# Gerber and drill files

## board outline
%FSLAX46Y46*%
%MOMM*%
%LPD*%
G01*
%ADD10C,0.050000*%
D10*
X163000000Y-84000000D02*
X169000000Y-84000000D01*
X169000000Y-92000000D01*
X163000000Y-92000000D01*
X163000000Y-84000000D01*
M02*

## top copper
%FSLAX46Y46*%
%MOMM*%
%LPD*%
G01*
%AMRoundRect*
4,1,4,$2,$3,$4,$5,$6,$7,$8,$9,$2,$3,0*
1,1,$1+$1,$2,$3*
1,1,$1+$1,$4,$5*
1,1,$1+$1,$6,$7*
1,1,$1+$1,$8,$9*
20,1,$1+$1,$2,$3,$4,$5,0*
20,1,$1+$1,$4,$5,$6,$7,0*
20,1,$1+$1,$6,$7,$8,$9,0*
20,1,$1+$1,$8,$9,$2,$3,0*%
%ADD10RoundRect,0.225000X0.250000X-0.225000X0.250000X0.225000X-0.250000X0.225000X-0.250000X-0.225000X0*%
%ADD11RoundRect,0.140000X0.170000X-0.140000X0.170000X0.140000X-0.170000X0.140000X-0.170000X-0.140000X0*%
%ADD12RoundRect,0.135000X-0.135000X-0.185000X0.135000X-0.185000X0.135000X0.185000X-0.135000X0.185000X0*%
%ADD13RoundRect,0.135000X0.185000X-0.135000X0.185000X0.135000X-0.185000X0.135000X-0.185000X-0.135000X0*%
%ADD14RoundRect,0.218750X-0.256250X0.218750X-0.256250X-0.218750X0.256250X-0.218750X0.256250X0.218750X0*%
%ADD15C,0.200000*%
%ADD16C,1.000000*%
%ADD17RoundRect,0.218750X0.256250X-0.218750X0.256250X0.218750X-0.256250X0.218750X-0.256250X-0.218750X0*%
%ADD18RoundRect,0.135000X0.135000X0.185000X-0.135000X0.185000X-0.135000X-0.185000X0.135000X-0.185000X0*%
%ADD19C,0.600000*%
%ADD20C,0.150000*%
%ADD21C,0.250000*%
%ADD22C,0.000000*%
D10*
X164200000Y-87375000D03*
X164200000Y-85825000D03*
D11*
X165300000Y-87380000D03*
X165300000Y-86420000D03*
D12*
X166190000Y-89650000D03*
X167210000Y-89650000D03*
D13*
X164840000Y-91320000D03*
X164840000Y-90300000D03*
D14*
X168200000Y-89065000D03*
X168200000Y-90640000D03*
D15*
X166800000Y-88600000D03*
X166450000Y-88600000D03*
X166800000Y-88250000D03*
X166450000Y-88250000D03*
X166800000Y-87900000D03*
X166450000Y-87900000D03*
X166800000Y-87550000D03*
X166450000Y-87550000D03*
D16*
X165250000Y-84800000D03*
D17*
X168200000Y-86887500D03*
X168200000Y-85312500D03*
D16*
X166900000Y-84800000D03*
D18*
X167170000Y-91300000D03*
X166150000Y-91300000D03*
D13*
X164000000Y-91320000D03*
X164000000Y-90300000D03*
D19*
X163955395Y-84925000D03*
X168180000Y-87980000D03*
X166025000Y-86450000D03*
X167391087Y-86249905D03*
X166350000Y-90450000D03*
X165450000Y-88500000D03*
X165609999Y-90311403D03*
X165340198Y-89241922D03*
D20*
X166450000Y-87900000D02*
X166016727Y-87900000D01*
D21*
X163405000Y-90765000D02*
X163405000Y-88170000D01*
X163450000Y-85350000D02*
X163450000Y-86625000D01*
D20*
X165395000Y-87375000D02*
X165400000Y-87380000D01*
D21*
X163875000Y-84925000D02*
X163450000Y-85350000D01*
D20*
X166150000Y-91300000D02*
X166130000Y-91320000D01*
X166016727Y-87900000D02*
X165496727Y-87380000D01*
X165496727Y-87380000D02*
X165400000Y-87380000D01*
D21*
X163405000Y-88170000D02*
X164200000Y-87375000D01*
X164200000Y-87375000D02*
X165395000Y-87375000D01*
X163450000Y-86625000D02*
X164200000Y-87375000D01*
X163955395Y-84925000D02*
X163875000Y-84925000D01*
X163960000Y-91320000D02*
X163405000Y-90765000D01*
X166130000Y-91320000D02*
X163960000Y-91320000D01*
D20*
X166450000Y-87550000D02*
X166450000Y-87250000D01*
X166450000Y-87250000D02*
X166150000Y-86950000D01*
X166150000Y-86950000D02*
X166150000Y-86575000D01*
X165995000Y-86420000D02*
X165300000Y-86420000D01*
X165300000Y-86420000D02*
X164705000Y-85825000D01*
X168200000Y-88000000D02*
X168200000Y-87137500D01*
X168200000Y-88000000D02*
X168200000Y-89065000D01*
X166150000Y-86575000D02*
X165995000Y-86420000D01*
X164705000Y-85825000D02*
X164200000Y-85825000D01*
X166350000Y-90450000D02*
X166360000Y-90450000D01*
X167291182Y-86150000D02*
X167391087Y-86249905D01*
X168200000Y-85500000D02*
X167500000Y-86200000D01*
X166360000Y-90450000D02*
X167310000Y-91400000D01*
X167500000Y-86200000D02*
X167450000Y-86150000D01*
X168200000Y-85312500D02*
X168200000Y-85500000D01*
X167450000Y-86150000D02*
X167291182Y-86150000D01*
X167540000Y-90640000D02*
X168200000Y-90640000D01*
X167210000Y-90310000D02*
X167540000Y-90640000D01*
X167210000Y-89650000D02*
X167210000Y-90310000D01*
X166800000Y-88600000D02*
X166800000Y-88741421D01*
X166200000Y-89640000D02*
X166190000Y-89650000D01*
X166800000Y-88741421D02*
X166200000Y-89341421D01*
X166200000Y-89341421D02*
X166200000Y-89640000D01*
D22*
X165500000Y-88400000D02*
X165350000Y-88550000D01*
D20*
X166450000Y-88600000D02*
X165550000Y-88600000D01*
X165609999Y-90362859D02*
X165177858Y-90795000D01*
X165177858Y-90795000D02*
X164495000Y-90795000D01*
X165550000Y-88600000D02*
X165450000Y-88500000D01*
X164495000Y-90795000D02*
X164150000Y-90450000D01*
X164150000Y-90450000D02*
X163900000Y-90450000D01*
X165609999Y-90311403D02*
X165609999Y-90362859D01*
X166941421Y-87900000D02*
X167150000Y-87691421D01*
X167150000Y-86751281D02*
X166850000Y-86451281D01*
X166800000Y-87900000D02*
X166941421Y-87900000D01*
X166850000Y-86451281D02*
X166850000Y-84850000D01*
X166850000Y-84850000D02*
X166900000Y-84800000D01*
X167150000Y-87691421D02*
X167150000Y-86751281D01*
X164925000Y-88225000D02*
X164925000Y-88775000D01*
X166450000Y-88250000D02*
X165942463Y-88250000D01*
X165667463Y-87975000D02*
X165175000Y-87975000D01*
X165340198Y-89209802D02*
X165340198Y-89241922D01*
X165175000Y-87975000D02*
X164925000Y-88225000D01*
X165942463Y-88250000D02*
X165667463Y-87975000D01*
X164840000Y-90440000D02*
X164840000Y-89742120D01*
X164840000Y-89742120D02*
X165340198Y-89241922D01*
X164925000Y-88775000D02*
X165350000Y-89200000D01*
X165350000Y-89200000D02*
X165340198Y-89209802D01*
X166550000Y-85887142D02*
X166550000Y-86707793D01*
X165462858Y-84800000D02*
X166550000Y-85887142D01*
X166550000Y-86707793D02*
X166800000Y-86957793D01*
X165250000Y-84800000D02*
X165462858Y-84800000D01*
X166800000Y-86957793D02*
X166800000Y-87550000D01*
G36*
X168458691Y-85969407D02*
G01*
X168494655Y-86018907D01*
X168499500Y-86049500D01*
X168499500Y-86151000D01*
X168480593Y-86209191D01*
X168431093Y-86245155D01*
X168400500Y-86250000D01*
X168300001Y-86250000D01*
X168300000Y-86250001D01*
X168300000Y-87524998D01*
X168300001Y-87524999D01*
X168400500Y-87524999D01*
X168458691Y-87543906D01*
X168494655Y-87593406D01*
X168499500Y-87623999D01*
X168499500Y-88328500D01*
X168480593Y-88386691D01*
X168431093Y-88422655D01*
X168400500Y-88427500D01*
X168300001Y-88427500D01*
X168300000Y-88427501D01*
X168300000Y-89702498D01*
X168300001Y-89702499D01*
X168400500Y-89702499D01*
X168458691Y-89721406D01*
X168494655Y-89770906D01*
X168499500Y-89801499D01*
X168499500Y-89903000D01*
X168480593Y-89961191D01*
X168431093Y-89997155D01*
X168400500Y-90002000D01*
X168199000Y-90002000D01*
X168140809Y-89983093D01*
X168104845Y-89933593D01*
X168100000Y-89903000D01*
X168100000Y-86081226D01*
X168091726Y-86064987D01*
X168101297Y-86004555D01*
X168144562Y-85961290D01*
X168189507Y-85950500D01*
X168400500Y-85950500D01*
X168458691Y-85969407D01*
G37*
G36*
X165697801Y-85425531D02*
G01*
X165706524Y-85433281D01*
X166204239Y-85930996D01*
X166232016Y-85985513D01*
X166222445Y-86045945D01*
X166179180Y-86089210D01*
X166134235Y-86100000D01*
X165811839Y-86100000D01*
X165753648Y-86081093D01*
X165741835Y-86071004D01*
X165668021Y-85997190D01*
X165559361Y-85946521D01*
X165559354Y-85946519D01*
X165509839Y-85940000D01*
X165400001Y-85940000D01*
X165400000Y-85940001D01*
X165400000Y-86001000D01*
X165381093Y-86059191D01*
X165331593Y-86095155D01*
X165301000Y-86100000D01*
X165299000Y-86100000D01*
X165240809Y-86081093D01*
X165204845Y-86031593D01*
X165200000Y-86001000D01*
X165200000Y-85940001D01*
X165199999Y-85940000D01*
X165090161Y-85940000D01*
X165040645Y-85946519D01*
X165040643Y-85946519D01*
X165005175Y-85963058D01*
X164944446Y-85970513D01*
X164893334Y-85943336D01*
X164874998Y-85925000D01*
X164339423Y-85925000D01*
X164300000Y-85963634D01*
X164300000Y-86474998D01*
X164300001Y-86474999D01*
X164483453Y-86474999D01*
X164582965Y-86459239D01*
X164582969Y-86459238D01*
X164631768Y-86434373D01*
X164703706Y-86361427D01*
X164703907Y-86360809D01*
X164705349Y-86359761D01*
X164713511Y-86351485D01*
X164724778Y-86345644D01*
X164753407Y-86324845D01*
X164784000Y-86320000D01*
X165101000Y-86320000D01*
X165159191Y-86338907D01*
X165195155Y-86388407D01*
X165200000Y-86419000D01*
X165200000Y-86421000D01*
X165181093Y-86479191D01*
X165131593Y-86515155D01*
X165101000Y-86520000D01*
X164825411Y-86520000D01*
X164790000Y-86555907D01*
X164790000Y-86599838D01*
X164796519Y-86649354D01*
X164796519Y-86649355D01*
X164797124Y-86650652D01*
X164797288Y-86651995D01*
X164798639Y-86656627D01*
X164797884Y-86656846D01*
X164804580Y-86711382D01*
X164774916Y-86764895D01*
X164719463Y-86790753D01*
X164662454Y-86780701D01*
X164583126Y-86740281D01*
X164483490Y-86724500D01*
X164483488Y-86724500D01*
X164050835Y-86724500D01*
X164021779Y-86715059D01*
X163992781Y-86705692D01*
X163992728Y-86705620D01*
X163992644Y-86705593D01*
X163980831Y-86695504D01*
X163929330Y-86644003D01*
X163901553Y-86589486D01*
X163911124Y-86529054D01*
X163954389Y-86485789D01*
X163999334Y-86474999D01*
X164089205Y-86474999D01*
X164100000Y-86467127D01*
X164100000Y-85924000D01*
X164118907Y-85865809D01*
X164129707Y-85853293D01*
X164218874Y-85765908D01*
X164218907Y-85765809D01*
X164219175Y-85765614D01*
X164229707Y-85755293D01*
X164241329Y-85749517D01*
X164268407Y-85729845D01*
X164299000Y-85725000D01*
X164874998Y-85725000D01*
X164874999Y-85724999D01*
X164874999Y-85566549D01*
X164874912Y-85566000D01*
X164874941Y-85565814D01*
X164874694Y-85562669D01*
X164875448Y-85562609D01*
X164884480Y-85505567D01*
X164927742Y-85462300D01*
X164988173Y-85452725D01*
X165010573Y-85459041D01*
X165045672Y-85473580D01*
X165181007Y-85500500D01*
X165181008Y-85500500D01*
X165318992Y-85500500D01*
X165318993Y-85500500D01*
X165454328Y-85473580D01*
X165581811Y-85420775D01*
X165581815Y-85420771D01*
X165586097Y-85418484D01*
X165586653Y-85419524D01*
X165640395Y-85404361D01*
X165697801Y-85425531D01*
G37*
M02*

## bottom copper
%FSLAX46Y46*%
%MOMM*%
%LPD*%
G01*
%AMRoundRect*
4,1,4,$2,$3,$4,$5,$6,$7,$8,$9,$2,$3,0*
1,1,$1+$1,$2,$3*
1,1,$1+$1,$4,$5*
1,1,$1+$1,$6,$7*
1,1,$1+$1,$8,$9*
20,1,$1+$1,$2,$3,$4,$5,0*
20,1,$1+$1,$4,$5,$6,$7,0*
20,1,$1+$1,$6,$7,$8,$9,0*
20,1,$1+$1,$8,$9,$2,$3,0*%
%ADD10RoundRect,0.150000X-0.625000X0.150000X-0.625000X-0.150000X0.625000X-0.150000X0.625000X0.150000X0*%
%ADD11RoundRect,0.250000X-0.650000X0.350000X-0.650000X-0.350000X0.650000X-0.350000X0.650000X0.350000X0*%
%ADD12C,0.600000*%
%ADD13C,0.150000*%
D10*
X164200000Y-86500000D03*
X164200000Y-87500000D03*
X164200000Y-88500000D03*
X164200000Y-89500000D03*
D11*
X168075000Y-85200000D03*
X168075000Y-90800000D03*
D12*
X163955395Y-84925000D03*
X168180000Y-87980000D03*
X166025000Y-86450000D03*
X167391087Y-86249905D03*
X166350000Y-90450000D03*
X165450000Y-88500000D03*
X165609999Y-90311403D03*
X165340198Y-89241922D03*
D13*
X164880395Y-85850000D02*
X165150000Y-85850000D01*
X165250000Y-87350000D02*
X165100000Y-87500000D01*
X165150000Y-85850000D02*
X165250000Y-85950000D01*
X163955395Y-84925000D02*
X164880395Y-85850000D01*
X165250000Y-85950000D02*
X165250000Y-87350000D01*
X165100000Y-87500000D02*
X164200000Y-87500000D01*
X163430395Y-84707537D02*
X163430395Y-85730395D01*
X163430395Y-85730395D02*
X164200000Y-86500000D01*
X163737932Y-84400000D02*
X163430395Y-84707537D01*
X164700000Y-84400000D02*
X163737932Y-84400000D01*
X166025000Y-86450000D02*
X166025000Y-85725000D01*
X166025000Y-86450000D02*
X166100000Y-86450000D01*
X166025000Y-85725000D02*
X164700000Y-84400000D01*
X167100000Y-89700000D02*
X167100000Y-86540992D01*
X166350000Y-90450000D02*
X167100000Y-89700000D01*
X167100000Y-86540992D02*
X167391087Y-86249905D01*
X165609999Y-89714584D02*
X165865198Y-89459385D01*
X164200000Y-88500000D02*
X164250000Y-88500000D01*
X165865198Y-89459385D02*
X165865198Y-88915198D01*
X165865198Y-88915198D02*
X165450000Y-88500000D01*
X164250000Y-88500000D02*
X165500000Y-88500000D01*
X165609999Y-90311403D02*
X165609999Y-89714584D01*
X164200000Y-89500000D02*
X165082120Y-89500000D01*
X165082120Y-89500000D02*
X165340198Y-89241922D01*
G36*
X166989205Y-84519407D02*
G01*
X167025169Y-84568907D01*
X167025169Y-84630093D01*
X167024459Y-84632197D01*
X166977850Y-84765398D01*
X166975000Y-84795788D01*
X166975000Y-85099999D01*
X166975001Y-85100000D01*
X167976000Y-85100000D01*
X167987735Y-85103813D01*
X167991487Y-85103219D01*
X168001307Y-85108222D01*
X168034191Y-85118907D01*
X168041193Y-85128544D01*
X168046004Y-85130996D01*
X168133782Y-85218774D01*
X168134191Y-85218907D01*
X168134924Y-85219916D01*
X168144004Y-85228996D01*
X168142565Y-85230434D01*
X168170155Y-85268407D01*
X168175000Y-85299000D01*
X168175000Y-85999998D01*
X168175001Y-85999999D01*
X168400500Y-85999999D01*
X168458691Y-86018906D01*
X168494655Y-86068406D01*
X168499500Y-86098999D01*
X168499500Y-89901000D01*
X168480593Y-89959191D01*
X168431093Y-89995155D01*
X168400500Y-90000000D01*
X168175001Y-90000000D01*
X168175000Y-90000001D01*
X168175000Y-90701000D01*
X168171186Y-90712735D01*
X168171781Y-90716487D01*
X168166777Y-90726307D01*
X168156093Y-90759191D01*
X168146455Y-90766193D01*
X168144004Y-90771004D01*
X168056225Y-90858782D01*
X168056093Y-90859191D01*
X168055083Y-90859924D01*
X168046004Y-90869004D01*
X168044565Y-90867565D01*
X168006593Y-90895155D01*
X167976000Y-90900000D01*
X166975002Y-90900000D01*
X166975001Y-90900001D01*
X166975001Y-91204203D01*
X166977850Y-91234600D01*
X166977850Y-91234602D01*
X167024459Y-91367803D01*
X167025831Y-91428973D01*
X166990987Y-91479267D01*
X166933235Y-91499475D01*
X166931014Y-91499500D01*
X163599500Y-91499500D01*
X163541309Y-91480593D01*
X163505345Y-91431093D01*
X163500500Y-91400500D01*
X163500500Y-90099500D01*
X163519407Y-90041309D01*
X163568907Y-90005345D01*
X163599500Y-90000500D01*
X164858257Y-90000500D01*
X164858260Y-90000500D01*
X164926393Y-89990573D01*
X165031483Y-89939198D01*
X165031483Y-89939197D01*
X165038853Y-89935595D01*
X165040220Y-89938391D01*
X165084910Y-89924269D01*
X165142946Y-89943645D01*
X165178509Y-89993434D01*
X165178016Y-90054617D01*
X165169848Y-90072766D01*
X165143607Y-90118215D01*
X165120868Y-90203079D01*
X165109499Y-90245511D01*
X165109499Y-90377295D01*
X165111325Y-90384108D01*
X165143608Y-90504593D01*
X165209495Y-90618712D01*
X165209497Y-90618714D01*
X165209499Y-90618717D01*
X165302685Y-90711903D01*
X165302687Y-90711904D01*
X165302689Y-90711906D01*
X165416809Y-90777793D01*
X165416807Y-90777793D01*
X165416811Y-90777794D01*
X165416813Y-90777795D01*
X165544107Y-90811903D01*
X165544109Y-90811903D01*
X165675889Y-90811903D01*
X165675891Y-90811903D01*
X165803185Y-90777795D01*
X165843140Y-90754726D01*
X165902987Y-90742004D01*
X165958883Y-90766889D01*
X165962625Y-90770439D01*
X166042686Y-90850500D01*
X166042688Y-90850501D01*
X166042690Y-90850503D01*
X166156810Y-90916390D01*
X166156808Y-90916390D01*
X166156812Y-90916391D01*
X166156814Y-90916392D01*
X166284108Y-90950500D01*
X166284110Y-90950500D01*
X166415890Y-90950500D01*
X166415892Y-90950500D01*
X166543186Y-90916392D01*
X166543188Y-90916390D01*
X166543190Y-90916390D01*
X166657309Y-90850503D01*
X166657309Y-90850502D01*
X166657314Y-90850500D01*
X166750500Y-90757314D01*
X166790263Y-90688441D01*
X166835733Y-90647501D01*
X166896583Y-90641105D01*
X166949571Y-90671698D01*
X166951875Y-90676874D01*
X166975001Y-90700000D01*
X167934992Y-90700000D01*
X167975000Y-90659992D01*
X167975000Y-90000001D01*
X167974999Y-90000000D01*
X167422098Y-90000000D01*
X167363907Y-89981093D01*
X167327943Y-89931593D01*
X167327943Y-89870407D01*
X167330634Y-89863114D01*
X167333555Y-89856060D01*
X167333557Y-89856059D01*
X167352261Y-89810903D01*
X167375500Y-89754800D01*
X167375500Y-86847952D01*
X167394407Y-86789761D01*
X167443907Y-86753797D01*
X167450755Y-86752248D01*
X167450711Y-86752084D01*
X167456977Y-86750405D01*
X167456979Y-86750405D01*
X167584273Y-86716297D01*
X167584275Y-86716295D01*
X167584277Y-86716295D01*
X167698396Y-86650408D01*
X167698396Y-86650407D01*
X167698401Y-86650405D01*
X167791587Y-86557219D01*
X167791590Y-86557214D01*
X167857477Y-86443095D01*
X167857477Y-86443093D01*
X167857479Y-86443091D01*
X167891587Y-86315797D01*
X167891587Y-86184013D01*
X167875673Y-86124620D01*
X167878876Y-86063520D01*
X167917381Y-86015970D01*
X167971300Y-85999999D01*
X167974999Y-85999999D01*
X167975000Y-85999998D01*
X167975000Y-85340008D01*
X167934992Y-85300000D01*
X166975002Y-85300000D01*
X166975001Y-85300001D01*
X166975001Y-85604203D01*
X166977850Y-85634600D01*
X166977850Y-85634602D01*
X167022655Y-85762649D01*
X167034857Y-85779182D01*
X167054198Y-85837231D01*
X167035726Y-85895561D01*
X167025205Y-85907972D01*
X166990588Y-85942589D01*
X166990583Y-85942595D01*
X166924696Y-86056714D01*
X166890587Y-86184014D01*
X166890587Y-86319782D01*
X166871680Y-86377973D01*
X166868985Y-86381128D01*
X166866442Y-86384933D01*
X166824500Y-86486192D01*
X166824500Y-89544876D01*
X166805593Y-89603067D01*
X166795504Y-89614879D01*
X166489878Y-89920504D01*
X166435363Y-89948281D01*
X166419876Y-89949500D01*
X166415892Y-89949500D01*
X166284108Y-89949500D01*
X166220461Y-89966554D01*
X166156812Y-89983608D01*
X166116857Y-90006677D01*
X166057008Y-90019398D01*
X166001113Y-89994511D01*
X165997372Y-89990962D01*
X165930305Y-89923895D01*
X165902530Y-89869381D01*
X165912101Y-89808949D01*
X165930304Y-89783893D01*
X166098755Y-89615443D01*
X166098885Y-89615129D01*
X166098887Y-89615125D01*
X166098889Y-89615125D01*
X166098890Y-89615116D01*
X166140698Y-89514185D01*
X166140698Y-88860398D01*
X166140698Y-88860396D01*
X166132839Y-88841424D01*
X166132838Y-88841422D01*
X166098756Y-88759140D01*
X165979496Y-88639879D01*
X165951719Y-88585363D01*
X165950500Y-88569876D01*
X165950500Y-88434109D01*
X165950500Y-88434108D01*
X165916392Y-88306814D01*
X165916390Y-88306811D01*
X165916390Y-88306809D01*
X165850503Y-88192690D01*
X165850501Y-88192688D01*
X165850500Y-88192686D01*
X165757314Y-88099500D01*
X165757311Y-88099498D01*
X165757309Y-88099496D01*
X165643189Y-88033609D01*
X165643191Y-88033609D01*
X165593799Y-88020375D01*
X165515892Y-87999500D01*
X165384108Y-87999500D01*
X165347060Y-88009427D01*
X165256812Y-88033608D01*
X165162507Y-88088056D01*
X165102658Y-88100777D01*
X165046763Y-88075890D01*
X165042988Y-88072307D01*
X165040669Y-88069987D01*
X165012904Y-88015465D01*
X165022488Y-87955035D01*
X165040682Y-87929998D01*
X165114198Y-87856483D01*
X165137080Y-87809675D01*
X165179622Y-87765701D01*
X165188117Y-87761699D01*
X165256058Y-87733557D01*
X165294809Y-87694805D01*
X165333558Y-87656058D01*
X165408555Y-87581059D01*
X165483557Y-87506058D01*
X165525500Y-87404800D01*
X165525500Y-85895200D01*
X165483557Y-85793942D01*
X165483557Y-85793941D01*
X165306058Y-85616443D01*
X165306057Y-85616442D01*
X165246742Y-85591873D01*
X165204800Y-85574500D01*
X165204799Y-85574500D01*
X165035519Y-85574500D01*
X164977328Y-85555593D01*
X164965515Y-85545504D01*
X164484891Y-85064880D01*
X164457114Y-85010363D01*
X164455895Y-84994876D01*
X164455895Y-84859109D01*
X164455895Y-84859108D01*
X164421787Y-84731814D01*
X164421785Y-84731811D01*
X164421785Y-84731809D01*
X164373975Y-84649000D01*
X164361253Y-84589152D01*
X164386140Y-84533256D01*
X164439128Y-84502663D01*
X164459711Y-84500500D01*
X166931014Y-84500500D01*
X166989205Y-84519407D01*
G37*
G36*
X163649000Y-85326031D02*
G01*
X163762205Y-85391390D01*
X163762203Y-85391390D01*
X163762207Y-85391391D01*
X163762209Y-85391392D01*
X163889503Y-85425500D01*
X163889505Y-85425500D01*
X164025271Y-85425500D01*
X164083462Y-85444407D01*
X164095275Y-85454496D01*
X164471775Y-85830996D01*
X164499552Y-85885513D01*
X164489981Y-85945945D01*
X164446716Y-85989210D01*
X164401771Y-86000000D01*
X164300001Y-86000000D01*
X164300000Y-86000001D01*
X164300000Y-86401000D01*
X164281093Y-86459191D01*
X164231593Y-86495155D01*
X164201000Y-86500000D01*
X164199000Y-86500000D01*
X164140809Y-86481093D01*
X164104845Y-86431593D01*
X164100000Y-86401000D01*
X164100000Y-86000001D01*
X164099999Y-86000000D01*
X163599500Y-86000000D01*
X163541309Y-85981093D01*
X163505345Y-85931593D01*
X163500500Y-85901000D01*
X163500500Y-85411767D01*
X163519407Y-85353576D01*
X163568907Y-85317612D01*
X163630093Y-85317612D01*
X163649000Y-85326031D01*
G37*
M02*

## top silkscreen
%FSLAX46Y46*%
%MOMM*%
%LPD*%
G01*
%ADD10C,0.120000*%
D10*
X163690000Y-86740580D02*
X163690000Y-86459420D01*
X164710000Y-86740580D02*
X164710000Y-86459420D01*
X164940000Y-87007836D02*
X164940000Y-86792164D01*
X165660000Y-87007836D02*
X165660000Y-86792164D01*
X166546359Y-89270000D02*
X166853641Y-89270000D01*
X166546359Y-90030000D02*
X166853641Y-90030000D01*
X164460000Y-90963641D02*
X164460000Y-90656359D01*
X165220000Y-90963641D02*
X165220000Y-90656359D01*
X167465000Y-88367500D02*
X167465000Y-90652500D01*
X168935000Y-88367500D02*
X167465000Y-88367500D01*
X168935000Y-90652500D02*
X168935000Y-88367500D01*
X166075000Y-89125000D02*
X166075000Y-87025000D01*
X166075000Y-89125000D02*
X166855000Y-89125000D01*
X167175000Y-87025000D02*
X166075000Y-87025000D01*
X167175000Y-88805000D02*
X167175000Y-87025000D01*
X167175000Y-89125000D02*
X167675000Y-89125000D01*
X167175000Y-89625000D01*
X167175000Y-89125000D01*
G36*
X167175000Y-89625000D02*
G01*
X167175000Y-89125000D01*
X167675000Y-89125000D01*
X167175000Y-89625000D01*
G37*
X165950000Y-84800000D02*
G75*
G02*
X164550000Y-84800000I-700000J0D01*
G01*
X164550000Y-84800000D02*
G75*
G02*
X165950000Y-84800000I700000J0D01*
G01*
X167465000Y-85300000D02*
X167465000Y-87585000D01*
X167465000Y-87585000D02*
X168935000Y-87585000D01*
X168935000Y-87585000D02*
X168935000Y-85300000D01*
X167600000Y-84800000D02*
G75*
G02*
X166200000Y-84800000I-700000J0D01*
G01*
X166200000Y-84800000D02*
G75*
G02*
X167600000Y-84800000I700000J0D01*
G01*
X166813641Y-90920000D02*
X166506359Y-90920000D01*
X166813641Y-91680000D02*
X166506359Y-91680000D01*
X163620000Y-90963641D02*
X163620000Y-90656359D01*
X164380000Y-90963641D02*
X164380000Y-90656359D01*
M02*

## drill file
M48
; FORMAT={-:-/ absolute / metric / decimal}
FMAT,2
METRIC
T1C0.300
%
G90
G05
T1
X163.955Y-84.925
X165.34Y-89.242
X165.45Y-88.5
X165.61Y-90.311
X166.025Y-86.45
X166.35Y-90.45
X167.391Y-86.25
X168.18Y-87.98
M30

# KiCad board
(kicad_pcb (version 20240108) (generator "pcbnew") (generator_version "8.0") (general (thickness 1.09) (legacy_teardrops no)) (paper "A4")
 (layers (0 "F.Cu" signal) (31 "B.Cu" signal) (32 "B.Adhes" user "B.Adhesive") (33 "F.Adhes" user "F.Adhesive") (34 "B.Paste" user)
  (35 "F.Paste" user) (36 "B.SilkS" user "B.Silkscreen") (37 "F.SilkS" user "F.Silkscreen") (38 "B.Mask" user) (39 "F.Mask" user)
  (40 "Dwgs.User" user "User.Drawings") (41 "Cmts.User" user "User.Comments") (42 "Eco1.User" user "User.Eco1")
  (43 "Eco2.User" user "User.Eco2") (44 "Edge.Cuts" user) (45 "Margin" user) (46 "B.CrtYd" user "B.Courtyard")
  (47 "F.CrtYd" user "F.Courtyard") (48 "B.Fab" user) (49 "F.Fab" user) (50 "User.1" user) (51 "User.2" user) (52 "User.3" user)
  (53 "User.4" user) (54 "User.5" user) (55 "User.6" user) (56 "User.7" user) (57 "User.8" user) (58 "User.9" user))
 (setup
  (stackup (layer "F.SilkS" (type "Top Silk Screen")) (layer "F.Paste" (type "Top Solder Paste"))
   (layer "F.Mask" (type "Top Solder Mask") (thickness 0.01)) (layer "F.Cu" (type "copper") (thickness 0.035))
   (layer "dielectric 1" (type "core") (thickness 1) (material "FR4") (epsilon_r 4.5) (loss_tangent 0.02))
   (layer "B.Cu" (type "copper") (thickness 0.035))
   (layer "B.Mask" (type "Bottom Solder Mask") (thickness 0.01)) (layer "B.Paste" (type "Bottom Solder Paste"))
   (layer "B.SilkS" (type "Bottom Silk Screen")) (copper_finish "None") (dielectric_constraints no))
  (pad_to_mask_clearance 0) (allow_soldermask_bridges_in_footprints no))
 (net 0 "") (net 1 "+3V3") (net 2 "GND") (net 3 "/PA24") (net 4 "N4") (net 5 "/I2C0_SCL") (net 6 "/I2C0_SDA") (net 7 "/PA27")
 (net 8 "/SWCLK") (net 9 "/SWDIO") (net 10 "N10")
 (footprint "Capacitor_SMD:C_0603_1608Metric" (layer "F.Cu") (at 164.2 86.6 90)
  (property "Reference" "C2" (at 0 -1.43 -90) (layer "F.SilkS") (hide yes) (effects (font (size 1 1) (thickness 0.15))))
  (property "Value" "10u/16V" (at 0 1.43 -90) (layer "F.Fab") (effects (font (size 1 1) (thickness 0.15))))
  (fp_line (start -0.14058 -0.51) (end 0.14058 -0.51) (stroke (width 0.12) (type solid)) (layer "F.SilkS"))
  (fp_line (start -0.14058 0.51) (end 0.14058 0.51) (stroke (width 0.12) (type solid)) (layer "F.SilkS"))
  (pad "1" smd roundrect (at -0.775 0 90) (size 0.9 0.95) (layers "F.Cu" "F.Paste" "F.Mask") (roundrect_rratio 0.25) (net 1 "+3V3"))
  (pad "2" smd roundrect (at 0.775 0 90) (size 0.9 0.95) (layers "F.Cu" "F.Paste" "F.Mask") (roundrect_rratio 0.25) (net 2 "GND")))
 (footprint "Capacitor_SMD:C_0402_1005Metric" (layer "F.Cu") (at 165.3 86.9 90)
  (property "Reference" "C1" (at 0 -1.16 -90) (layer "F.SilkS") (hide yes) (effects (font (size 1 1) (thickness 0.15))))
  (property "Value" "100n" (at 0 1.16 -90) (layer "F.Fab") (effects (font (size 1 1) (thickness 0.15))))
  (fp_line (start -0.107836 -0.36) (end 0.107836 -0.36) (stroke (width 0.12) (type solid)) (layer "F.SilkS"))
  (fp_line (start -0.107836 0.36) (end 0.107836 0.36) (stroke (width 0.12) (type solid)) (layer "F.SilkS"))
  (pad "1" smd roundrect (at -0.48 0 90) (size 0.56 0.62) (layers "F.Cu" "F.Paste" "F.Mask") (roundrect_rratio 0.25) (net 1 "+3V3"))
  (pad "2" smd roundrect (at 0.48 0 90) (size 0.56 0.62) (layers "F.Cu" "F.Paste" "F.Mask") (roundrect_rratio 0.25) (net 2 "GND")))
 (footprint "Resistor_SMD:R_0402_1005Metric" (layer "F.Cu") (at 166.7 89.65)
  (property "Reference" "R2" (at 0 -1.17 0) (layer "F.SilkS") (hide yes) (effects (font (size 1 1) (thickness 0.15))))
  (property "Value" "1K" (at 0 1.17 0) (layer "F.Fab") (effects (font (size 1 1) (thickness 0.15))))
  (fp_line (start -0.153641 -0.38) (end 0.153641 -0.38) (stroke (width 0.12) (type solid)) (layer "F.SilkS"))
  (fp_line (start -0.153641 0.38) (end 0.153641 0.38) (stroke (width 0.12) (type solid)) (layer "F.SilkS"))
  (pad "1" smd roundrect (at -0.51 0) (size 0.54 0.64) (layers "F.Cu" "F.Paste" "F.Mask") (roundrect_rratio 0.25) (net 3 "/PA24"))
  (pad "2" smd roundrect (at 0.51 0) (size 0.54 0.64) (layers "F.Cu" "F.Paste" "F.Mask") (roundrect_rratio 0.25) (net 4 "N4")))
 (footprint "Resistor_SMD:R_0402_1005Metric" (layer "F.Cu") (at 164.84 90.81 90)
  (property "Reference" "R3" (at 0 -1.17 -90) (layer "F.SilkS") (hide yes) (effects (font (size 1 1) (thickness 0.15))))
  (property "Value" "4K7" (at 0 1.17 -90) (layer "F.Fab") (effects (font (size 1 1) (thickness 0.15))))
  (fp_line (start -0.153641 -0.38) (end 0.153641 -0.38) (stroke (width 0.12) (type solid)) (layer "F.SilkS"))
  (fp_line (start -0.153641 0.38) (end 0.153641 0.38) (stroke (width 0.12) (type solid)) (layer "F.SilkS"))
  (pad "1" smd roundrect (at -0.51 0 90) (size 0.54 0.64) (layers "F.Cu" "F.Paste" "F.Mask") (roundrect_rratio 0.25) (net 1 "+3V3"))
  (pad "2" smd roundrect (at 0.51 0 90) (size 0.54 0.64) (layers "F.Cu" "F.Paste" "F.Mask") (roundrect_rratio 0.25) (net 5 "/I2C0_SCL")))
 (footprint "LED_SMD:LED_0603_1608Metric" (layer "F.Cu") (at 168.2 89.8525 -90)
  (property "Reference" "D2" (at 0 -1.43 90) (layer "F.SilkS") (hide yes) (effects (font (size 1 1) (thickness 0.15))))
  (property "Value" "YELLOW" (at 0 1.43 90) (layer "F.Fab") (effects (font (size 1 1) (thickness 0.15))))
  (fp_line (start -1.485 0.735) (end 0.8 0.735) (stroke (width 0.12) (type solid)) (layer "F.SilkS"))
  (fp_line (start -1.485 -0.735) (end -1.485 0.735) (stroke (width 0.12) (type solid)) (layer "F.SilkS"))
  (fp_line (start 0.8 -0.735) (end -1.485 -0.735) (stroke (width 0.12) (type solid)) (layer "F.SilkS"))
  (pad "1" smd roundrect (at -0.7875 0 270) (size 0.875 0.95) (layers "F.Cu" "F.Paste" "F.Mask") (roundrect_rratio 0.25) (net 2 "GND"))
  (pad "2" smd roundrect (at 0.7875 0 270) (size 0.875 0.95) (layers "F.Cu" "F.Paste" "F.Mask") (roundrect_rratio 0.25) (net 4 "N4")))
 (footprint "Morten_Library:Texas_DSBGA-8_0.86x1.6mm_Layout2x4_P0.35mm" (layer "F.Cu") (at 166.625 88.075 180)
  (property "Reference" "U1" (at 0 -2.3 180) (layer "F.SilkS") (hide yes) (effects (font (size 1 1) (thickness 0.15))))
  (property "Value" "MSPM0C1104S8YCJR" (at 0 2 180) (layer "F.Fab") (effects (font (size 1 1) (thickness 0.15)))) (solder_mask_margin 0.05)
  (fp_line (start 0.55 -1.05) (end 0.55 1.05) (stroke (width 0.12) (type solid)) (layer "F.SilkS"))
  (fp_line (start 0.55 -1.05) (end -0.23 -1.05) (stroke (width 0.12) (type solid)) (layer "F.SilkS"))
  (fp_line (start -0.55 1.05) (end 0.55 1.05) (stroke (width 0.12) (type solid)) (layer "F.SilkS"))
  (fp_line (start -0.55 -0.73) (end -0.55 1.05) (stroke (width 0.12) (type solid)) (layer "F.SilkS"))
  (fp_poly
   (pts (xy -0.55 -1.05) (xy -1.05 -1.05) (xy -0.55 -1.55) (xy -0.55 -1.05)) (stroke (width 0.12) (type solid)) (fill solid)
   (layer "F.SilkS"))
  (pad "" smd rect (at -0.175 -0.525 180) (size 0.25 0.25) (layers "F.Paste"))
  (pad "" smd rect (at -0.175 -0.175 180) (size 0.25 0.25) (layers "F.Paste"))
  (pad "" smd rect (at -0.175 0.175 180) (size 0.25 0.25) (layers "F.Paste"))
  (pad "" smd rect (at -0.175 0.525 180) (size 0.25 0.25) (layers "F.Paste"))
  (pad "" smd rect (at 0.175 -0.525 180) (size 0.25 0.25) (layers "F.Paste"))
  (pad "" smd rect (at 0.175 -0.175 180) (size 0.25 0.25) (layers "F.Paste"))
  (pad "" smd rect (at 0.175 0.175 180) (size 0.25 0.25) (layers "F.Paste"))
  (pad "" smd rect (at 0.175 0.525 180) (size 0.25 0.25) (layers "F.Paste"))
  (pad "A1" smd circle (at -0.175 -0.525 180) (size 0.2 0.2) (layers "F.Cu" "F.Mask") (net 3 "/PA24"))
  (pad "A2" smd circle (at 0.175 -0.525 180) (size 0.2 0.2) (layers "F.Cu" "F.Mask") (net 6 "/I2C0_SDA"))
  (pad "B1" smd circle (at -0.175 -0.175 180) (size 0.2 0.2) (layers "F.Cu" "F.Mask") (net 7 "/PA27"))
  (pad "B2" smd circle (at 0.175 -0.175 180) (size 0.2 0.2) (layers "F.Cu" "F.Mask") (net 5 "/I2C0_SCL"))
  (pad "C1" smd circle (at -0.175 0.175 180) (size 0.2 0.2) (layers "F.Cu" "F.Mask") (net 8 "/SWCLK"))
  (pad "C2" smd circle (at 0.175 0.175 180) (size 0.2 0.2) (layers "F.Cu" "F.Mask") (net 1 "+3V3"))
  (pad "D1" smd circle (at -0.175 0.525 180) (size 0.2 0.2) (layers "F.Cu" "F.Mask") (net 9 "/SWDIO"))
  (pad "D2" smd circle (at 0.175 0.525 180) (size 0.2 0.2) (layers "F.Cu" "F.Mask") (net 2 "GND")))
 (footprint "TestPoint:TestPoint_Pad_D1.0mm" (layer "F.Cu") (at 165.25 84.8)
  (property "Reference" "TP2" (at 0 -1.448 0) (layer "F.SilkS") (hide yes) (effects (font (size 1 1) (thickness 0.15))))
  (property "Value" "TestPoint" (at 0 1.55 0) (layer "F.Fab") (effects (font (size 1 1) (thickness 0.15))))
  (fp_circle (center 0 0) (end 0 0.7) (stroke (width 0.12) (type solid)) (fill none) (layer "F.SilkS"))
  (pad "1" smd circle (at 0 0) (size 1 1) (layers "F.Cu" "F.Mask") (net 9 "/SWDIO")))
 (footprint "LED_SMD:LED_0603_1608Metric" (layer "F.Cu") (at 168.2 86.1 90)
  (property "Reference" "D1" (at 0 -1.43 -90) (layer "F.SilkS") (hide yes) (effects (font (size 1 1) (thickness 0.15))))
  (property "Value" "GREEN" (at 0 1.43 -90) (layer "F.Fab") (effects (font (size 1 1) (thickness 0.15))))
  (fp_line (start 0.8 -0.735) (end -1.485 -0.735) (stroke (width 0.12) (type solid)) (layer "F.SilkS"))
  (fp_line (start -1.485 -0.735) (end -1.485 0.735) (stroke (width 0.12) (type solid)) (layer "F.SilkS"))
  (fp_line (start -1.485 0.735) (end 0.8 0.735) (stroke (width 0.12) (type solid)) (layer "F.SilkS"))
  (pad "1" smd roundrect (at -0.7875 0 90) (size 0.875 0.95) (layers "F.Cu" "F.Paste" "F.Mask") (roundrect_rratio 0.25) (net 2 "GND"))
  (pad "2" smd roundrect (at 0.7875 0 90) (size 0.875 0.95) (layers "F.Cu" "F.Paste" "F.Mask") (roundrect_rratio 0.25) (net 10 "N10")))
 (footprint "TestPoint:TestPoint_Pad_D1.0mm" (layer "F.Cu") (at 166.9 84.8)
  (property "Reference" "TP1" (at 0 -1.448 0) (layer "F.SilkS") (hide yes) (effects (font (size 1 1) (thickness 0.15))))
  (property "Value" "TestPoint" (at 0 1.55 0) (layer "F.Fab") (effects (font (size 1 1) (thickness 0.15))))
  (fp_circle (center 0 0) (end 0 0.7) (stroke (width 0.12) (type solid)) (fill none) (layer "F.SilkS"))
  (pad "1" smd circle (at 0 0) (size 1 1) (layers "F.Cu" "F.Mask") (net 8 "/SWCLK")))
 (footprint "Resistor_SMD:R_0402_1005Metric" (layer "F.Cu") (at 166.66 91.3 180)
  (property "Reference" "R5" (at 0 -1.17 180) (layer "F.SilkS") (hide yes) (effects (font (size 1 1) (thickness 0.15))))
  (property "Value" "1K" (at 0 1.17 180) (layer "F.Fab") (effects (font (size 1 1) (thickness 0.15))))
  (fp_line (start -0.153641 0.38) (end 0.153641 0.38) (stroke (width 0.12) (type solid)) (layer "F.SilkS"))
  (fp_line (start -0.153641 -0.38) (end 0.153641 -0.38) (stroke (width 0.12) (type solid)) (layer "F.SilkS"))
  (pad "1" smd roundrect (at -0.51 0 180) (size 0.54 0.64) (layers "F.Cu" "F.Paste" "F.Mask") (roundrect_rratio 0.25) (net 10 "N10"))
  (pad "2" smd roundrect (at 0.51 0 180) (size 0.54 0.64) (layers "F.Cu" "F.Paste" "F.Mask") (roundrect_rratio 0.25) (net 1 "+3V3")))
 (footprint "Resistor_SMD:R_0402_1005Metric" (layer "F.Cu") (at 164 90.81 90)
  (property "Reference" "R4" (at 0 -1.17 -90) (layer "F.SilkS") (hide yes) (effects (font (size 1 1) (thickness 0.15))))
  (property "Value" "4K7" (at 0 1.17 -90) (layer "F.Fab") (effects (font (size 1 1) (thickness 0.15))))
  (fp_line (start -0.153641 -0.38) (end 0.153641 -0.38) (stroke (width 0.12) (type solid)) (layer "F.SilkS"))
  (fp_line (start -0.153641 0.38) (end 0.153641 0.38) (stroke (width 0.12) (type solid)) (layer "F.SilkS"))
  (pad "1" smd roundrect (at -0.51 0 90) (size 0.54 0.64) (layers "F.Cu" "F.Paste" "F.Mask") (roundrect_rratio 0.25) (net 1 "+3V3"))
  (pad "2" smd roundrect (at 0.51 0 90) (size 0.54 0.64) (layers "F.Cu" "F.Paste" "F.Mask") (roundrect_rratio 0.25) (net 6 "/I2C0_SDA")))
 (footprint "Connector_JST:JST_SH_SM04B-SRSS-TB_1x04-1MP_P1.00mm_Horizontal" (layer "B.Cu") (at 166.2 88 -90)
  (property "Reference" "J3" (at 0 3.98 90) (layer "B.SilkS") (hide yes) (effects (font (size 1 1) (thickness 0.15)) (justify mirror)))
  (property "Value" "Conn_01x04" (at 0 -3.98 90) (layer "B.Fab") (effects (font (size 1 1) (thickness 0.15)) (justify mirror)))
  (pad "1" smd roundrect (at -1.5 2 270) (size 0.6 1.55) (layers "B.Cu" "B.Paste" "B.Mask") (roundrect_rratio 0.25) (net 2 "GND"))
  (pad "2" smd roundrect (at -0.5 2 270) (size 0.6 1.55) (layers "B.Cu" "B.Paste" "B.Mask") (roundrect_rratio 0.25) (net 1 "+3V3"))
  (pad "3" smd roundrect (at 0.5 2 270) (size 0.6 1.55) (layers "B.Cu" "B.Paste" "B.Mask") (roundrect_rratio 0.25) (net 6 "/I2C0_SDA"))
  (pad "4" smd roundrect (at 1.5 2 270) (size 0.6 1.55) (layers "B.Cu" "B.Paste" "B.Mask") (roundrect_rratio 0.25) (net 5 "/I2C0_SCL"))
  (pad "MP" smd roundrect (at -2.8 -1.875 270) (size 1.2 1.8) (layers "B.Cu" "B.Paste" "B.Mask") (roundrect_rratio 0.2083333333)
   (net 2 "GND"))
  (pad "MP" smd roundrect (at 2.8 -1.875 270) (size 1.2 1.8) (layers "B.Cu" "B.Paste" "B.Mask") (roundrect_rratio 0.2083333333)
   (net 2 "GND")))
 (gr_rect (start 163 84) (end 169 92) (stroke (width 0.05) (type default)) (fill none) (layer "Edge.Cuts"))
 (segment (start 166.45 87.9) (end 166.016727 87.9) (width 0.15) (layer "F.Cu") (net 1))
 (segment (start 163.405 90.765) (end 163.405 88.17) (width 0.25) (layer "F.Cu") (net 1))
 (segment (start 163.45 85.35) (end 163.45 86.625) (width 0.25) (layer "F.Cu") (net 1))
 (segment (start 165.395 87.375) (end 165.4 87.38) (width 0.15) (layer "F.Cu") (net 1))
 (segment (start 163.875 84.925) (end 163.45 85.35) (width 0.25) (layer "F.Cu") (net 1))
 (segment (start 166.15 91.3) (end 166.13 91.32) (width 0.15) (layer "F.Cu") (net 1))
 (segment (start 166.016727 87.9) (end 165.496727 87.38) (width 0.15) (layer "F.Cu") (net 1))
 (segment (start 165.496727 87.38) (end 165.4 87.38) (width 0.15) (layer "F.Cu") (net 1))
 (segment (start 163.405 88.17) (end 164.2 87.375) (width 0.25) (layer "F.Cu") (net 1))
 (segment (start 164.2 87.375) (end 165.395 87.375) (width 0.25) (layer "F.Cu") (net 1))
 (segment (start 163.45 86.625) (end 164.2 87.375) (width 0.25) (layer "F.Cu") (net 1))
 (segment (start 163.955395 84.925) (end 163.875 84.925) (width 0.25) (layer "F.Cu") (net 1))
 (segment (start 163.96 91.32) (end 163.405 90.765) (width 0.25) (layer "F.Cu") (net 1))
 (segment (start 166.13 91.32) (end 163.96 91.32) (width 0.25) (layer "F.Cu") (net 1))
 (via (at 163.955395 84.925) (size 0.6) (drill 0.3) (layers "F.Cu" "B.Cu") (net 1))
 (segment (start 164.880395 85.85) (end 165.15 85.85) (width 0.15) (layer "B.Cu") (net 1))
 (segment (start 165.25 87.35) (end 165.1 87.5) (width 0.15) (layer "B.Cu") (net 1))
 (segment (start 165.15 85.85) (end 165.25 85.95) (width 0.15) (layer "B.Cu") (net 1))
 (segment (start 163.955395 84.925) (end 164.880395 85.85) (width 0.15) (layer "B.Cu") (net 1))
 (segment (start 165.25 85.95) (end 165.25 87.35) (width 0.15) (layer "B.Cu") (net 1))
 (segment (start 165.1 87.5) (end 164.2 87.5) (width 0.15) (layer "B.Cu") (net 1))
 (segment (start 166.45 87.55) (end 166.45 87.25) (width 0.15) (layer "F.Cu") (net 2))
 (segment (start 166.45 87.25) (end 166.15 86.95) (width 0.15) (layer "F.Cu") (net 2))
 (segment (start 166.15 86.95) (end 166.15 86.575) (width 0.15) (layer "F.Cu") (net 2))
 (segment (start 165.995 86.42) (end 165.3 86.42) (width 0.15) (layer "F.Cu") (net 2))
 (segment (start 165.3 86.42) (end 164.705 85.825) (width 0.15) (layer "F.Cu") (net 2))
 (segment (start 168.2 88) (end 168.2 87.1375) (width 0.15) (layer "F.Cu") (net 2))
 (segment (start 168.2 88) (end 168.2 89.065) (width 0.15) (layer "F.Cu") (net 2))
 (segment (start 166.15 86.575) (end 165.995 86.42) (width 0.15) (layer "F.Cu") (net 2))
 (segment (start 164.705 85.825) (end 164.2 85.825) (width 0.15) (layer "F.Cu") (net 2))
 (via (at 168.18 87.98) (size 0.6) (drill 0.3) (layers "F.Cu" "B.Cu") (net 2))
 (via (at 166.025 86.45) (size 0.6) (drill 0.3) (layers "F.Cu" "B.Cu") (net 2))
 (segment (start 163.430395 84.707537) (end 163.430395 85.730395) (width 0.15) (layer "B.Cu") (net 2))
 (segment (start 163.430395 85.730395) (end 164.2 86.5) (width 0.15) (layer "B.Cu") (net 2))
 (segment (start 163.737932 84.4) (end 163.430395 84.707537) (width 0.15) (layer "B.Cu") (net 2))
 (segment (start 164.7 84.4) (end 163.737932 84.4) (width 0.15) (layer "B.Cu") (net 2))
 (segment (start 166.025 86.45) (end 166.025 85.725) (width 0.15) (layer "B.Cu") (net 2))
 (segment (start 166.025 86.45) (end 166.1 86.45) (width 0.15) (layer "B.Cu") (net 2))
 (segment (start 166.025 85.725) (end 164.7 84.4) (width 0.15) (layer "B.Cu") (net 2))
 (segment (start 166.35 90.45) (end 166.36 90.45) (width 0.15) (layer "F.Cu") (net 10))
 (segment (start 167.291182 86.15) (end 167.391087 86.249905) (width 0.15) (layer "F.Cu") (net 10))
 (segment (start 168.2 85.5) (end 167.5 86.2) (width 0.15) (layer "F.Cu") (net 10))
 (segment (start 166.36 90.45) (end 167.31 91.4) (width 0.15) (layer "F.Cu") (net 10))
 (segment (start 167.5 86.2) (end 167.45 86.15) (width 0.15) (layer "F.Cu") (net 10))
 (segment (start 168.2 85.3125) (end 168.2 85.5) (width 0.15) (layer "F.Cu") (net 10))
 (segment (start 167.45 86.15) (end 167.291182 86.15) (width 0.15) (layer "F.Cu") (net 10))
 (via (at 167.391087 86.249905) (size 0.6) (drill 0.3) (layers "F.Cu" "B.Cu") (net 10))
 (via (at 166.35 90.45) (size 0.6) (drill 0.3) (layers "F.Cu" "B.Cu") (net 10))
 (segment (start 167.1 89.7) (end 167.1 86.540992) (width 0.15) (layer "B.Cu") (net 10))
 (segment (start 166.35 90.45) (end 167.1 89.7) (width 0.15) (layer "B.Cu") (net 10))
 (segment (start 167.1 86.540992) (end 167.391087 86.249905) (width 0.15) (layer "B.Cu") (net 10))
 (segment (start 167.54 90.64) (end 168.2 90.64) (width 0.15) (layer "F.Cu") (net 4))
 (segment (start 167.21 90.31) (end 167.54 90.64) (width 0.15) (layer "F.Cu") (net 4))
 (segment (start 167.21 89.65) (end 167.21 90.31) (width 0.15) (layer "F.Cu") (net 4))
 (segment (start 166.8 88.6) (end 166.8 88.741421) (width 0.15) (layer "F.Cu") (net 3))
 (segment (start 166.2 89.64) (end 166.19 89.65) (width 0.15) (layer "F.Cu") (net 3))
 (segment (start 166.8 88.741421) (end 166.2 89.341421) (width 0.15) (layer "F.Cu") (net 3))
 (segment (start 166.2 89.341421) (end 166.2 89.64) (width 0.15) (layer "F.Cu") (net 3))
 (segment (start 165.5 88.4) (end 165.35 88.55) (width 0) (layer "F.Cu") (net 6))
 (segment (start 166.45 88.6) (end 165.55 88.6) (width 0.15) (layer "F.Cu") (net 6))
 (segment (start 165.609999 90.362859) (end 165.177858 90.795) (width 0.15) (layer "F.Cu") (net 6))
 (segment (start 165.177858 90.795) (end 164.495 90.795) (width 0.15) (layer "F.Cu") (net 6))
 (segment (start 165.55 88.6) (end 165.45 88.5) (width 0.15) (layer "F.Cu") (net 6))
 (segment (start 164.495 90.795) (end 164.15 90.45) (width 0.15) (layer "F.Cu") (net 6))
 (segment (start 164.15 90.45) (end 163.9 90.45) (width 0.15) (layer "F.Cu") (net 6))
 (segment (start 165.609999 90.311403) (end 165.609999 90.362859) (width 0.15) (layer "F.Cu") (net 6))
 (via (at 165.45 88.5) (size 0.6) (drill 0.3) (layers "F.Cu" "B.Cu") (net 6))
 (via (at 165.609999 90.311403) (size 0.6) (drill 0.3) (layers "F.Cu" "B.Cu") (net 6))
 (segment (start 165.609999 89.714584) (end 165.865198 89.459385) (width 0.15) (layer "B.Cu") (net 6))
 (segment (start 164.2 88.5) (end 164.25 88.5) (width 0.15) (layer "B.Cu") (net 6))
 (segment (start 165.865198 89.459385) (end 165.865198 88.915198) (width 0.15) (layer "B.Cu") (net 6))
 (segment (start 165.865198 88.915198) (end 165.45 88.5) (width 0.15) (layer "B.Cu") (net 6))
 (segment (start 164.25 88.5) (end 165.5 88.5) (width 0.15) (layer "B.Cu") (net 6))
 (segment (start 165.609999 90.311403) (end 165.609999 89.714584) (width 0.15) (layer "B.Cu") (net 6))
 (segment (start 166.941421 87.9) (end 167.15 87.691421) (width 0.15) (layer "F.Cu") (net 8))
 (segment (start 167.15 86.751281) (end 166.85 86.451281) (width 0.15) (layer "F.Cu") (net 8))
 (segment (start 166.8 87.9) (end 166.941421 87.9) (width 0.15) (layer "F.Cu") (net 8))
 (segment (start 166.85 86.451281) (end 166.85 84.85) (width 0.15) (layer "F.Cu") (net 8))
 (segment (start 166.85 84.85) (end 166.9 84.8) (width 0.15) (layer "F.Cu") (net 8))
 (segment (start 167.15 87.691421) (end 167.15 86.751281) (width 0.15) (layer "F.Cu") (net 8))
 (segment (start 164.925 88.225) (end 164.925 88.775) (width 0.15) (layer "F.Cu") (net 5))
 (segment (start 166.45 88.25) (end 165.942463 88.25) (width 0.15) (layer "F.Cu") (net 5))
 (segment (start 165.667463 87.975) (end 165.175 87.975) (width 0.15) (layer "F.Cu") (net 5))
 (segment (start 165.340198 89.209802) (end 165.340198 89.241922) (width 0.15) (layer "F.Cu") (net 5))
 (segment (start 165.175 87.975) (end 164.925 88.225) (width 0.15) (layer "F.Cu") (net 5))
 (segment (start 165.942463 88.25) (end 165.667463 87.975) (width 0.15) (layer "F.Cu") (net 5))
 (segment (start 164.84 90.44) (end 164.84 89.74212) (width 0.15) (layer "F.Cu") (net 5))
 (segment (start 164.84 89.74212) (end 165.340198 89.241922) (width 0.15) (layer "F.Cu") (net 5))
 (segment (start 164.925 88.775) (end 165.35 89.2) (width 0.15) (layer "F.Cu") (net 5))
 (segment (start 165.35 89.2) (end 165.340198 89.209802) (width 0.15) (layer "F.Cu") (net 5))
 (via (at 165.340198 89.241922) (size 0.6) (drill 0.3) (layers "F.Cu" "B.Cu") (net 5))
 (segment (start 164.2 89.5) (end 165.08212 89.5) (width 0.15) (layer "B.Cu") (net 5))
 (segment (start 165.08212 89.5) (end 165.340198 89.241922) (width 0.15) (layer "B.Cu") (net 5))
 (segment (start 166.55 85.887142) (end 166.55 86.707793) (width 0.15) (layer "F.Cu") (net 9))
 (segment (start 165.462858 84.8) (end 166.55 85.887142) (width 0.15) (layer "F.Cu") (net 9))
 (segment (start 166.55 86.707793) (end 166.8 86.957793) (width 0.15) (layer "F.Cu") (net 9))
 (segment (start 165.25 84.8) (end 165.462858 84.8) (width 0.15) (layer "F.Cu") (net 9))
 (segment (start 166.8 86.957793) (end 166.8 87.55) (width 0.15) (layer "F.Cu") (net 9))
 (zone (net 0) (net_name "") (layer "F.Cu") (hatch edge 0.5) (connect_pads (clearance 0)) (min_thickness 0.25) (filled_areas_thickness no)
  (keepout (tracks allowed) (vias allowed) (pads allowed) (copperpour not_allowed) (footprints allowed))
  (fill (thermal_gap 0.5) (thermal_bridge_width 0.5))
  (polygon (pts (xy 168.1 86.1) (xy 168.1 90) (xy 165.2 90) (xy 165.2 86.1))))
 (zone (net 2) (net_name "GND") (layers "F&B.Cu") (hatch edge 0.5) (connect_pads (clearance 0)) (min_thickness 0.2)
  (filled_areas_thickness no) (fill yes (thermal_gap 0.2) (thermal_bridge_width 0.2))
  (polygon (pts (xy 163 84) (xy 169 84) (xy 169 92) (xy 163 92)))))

